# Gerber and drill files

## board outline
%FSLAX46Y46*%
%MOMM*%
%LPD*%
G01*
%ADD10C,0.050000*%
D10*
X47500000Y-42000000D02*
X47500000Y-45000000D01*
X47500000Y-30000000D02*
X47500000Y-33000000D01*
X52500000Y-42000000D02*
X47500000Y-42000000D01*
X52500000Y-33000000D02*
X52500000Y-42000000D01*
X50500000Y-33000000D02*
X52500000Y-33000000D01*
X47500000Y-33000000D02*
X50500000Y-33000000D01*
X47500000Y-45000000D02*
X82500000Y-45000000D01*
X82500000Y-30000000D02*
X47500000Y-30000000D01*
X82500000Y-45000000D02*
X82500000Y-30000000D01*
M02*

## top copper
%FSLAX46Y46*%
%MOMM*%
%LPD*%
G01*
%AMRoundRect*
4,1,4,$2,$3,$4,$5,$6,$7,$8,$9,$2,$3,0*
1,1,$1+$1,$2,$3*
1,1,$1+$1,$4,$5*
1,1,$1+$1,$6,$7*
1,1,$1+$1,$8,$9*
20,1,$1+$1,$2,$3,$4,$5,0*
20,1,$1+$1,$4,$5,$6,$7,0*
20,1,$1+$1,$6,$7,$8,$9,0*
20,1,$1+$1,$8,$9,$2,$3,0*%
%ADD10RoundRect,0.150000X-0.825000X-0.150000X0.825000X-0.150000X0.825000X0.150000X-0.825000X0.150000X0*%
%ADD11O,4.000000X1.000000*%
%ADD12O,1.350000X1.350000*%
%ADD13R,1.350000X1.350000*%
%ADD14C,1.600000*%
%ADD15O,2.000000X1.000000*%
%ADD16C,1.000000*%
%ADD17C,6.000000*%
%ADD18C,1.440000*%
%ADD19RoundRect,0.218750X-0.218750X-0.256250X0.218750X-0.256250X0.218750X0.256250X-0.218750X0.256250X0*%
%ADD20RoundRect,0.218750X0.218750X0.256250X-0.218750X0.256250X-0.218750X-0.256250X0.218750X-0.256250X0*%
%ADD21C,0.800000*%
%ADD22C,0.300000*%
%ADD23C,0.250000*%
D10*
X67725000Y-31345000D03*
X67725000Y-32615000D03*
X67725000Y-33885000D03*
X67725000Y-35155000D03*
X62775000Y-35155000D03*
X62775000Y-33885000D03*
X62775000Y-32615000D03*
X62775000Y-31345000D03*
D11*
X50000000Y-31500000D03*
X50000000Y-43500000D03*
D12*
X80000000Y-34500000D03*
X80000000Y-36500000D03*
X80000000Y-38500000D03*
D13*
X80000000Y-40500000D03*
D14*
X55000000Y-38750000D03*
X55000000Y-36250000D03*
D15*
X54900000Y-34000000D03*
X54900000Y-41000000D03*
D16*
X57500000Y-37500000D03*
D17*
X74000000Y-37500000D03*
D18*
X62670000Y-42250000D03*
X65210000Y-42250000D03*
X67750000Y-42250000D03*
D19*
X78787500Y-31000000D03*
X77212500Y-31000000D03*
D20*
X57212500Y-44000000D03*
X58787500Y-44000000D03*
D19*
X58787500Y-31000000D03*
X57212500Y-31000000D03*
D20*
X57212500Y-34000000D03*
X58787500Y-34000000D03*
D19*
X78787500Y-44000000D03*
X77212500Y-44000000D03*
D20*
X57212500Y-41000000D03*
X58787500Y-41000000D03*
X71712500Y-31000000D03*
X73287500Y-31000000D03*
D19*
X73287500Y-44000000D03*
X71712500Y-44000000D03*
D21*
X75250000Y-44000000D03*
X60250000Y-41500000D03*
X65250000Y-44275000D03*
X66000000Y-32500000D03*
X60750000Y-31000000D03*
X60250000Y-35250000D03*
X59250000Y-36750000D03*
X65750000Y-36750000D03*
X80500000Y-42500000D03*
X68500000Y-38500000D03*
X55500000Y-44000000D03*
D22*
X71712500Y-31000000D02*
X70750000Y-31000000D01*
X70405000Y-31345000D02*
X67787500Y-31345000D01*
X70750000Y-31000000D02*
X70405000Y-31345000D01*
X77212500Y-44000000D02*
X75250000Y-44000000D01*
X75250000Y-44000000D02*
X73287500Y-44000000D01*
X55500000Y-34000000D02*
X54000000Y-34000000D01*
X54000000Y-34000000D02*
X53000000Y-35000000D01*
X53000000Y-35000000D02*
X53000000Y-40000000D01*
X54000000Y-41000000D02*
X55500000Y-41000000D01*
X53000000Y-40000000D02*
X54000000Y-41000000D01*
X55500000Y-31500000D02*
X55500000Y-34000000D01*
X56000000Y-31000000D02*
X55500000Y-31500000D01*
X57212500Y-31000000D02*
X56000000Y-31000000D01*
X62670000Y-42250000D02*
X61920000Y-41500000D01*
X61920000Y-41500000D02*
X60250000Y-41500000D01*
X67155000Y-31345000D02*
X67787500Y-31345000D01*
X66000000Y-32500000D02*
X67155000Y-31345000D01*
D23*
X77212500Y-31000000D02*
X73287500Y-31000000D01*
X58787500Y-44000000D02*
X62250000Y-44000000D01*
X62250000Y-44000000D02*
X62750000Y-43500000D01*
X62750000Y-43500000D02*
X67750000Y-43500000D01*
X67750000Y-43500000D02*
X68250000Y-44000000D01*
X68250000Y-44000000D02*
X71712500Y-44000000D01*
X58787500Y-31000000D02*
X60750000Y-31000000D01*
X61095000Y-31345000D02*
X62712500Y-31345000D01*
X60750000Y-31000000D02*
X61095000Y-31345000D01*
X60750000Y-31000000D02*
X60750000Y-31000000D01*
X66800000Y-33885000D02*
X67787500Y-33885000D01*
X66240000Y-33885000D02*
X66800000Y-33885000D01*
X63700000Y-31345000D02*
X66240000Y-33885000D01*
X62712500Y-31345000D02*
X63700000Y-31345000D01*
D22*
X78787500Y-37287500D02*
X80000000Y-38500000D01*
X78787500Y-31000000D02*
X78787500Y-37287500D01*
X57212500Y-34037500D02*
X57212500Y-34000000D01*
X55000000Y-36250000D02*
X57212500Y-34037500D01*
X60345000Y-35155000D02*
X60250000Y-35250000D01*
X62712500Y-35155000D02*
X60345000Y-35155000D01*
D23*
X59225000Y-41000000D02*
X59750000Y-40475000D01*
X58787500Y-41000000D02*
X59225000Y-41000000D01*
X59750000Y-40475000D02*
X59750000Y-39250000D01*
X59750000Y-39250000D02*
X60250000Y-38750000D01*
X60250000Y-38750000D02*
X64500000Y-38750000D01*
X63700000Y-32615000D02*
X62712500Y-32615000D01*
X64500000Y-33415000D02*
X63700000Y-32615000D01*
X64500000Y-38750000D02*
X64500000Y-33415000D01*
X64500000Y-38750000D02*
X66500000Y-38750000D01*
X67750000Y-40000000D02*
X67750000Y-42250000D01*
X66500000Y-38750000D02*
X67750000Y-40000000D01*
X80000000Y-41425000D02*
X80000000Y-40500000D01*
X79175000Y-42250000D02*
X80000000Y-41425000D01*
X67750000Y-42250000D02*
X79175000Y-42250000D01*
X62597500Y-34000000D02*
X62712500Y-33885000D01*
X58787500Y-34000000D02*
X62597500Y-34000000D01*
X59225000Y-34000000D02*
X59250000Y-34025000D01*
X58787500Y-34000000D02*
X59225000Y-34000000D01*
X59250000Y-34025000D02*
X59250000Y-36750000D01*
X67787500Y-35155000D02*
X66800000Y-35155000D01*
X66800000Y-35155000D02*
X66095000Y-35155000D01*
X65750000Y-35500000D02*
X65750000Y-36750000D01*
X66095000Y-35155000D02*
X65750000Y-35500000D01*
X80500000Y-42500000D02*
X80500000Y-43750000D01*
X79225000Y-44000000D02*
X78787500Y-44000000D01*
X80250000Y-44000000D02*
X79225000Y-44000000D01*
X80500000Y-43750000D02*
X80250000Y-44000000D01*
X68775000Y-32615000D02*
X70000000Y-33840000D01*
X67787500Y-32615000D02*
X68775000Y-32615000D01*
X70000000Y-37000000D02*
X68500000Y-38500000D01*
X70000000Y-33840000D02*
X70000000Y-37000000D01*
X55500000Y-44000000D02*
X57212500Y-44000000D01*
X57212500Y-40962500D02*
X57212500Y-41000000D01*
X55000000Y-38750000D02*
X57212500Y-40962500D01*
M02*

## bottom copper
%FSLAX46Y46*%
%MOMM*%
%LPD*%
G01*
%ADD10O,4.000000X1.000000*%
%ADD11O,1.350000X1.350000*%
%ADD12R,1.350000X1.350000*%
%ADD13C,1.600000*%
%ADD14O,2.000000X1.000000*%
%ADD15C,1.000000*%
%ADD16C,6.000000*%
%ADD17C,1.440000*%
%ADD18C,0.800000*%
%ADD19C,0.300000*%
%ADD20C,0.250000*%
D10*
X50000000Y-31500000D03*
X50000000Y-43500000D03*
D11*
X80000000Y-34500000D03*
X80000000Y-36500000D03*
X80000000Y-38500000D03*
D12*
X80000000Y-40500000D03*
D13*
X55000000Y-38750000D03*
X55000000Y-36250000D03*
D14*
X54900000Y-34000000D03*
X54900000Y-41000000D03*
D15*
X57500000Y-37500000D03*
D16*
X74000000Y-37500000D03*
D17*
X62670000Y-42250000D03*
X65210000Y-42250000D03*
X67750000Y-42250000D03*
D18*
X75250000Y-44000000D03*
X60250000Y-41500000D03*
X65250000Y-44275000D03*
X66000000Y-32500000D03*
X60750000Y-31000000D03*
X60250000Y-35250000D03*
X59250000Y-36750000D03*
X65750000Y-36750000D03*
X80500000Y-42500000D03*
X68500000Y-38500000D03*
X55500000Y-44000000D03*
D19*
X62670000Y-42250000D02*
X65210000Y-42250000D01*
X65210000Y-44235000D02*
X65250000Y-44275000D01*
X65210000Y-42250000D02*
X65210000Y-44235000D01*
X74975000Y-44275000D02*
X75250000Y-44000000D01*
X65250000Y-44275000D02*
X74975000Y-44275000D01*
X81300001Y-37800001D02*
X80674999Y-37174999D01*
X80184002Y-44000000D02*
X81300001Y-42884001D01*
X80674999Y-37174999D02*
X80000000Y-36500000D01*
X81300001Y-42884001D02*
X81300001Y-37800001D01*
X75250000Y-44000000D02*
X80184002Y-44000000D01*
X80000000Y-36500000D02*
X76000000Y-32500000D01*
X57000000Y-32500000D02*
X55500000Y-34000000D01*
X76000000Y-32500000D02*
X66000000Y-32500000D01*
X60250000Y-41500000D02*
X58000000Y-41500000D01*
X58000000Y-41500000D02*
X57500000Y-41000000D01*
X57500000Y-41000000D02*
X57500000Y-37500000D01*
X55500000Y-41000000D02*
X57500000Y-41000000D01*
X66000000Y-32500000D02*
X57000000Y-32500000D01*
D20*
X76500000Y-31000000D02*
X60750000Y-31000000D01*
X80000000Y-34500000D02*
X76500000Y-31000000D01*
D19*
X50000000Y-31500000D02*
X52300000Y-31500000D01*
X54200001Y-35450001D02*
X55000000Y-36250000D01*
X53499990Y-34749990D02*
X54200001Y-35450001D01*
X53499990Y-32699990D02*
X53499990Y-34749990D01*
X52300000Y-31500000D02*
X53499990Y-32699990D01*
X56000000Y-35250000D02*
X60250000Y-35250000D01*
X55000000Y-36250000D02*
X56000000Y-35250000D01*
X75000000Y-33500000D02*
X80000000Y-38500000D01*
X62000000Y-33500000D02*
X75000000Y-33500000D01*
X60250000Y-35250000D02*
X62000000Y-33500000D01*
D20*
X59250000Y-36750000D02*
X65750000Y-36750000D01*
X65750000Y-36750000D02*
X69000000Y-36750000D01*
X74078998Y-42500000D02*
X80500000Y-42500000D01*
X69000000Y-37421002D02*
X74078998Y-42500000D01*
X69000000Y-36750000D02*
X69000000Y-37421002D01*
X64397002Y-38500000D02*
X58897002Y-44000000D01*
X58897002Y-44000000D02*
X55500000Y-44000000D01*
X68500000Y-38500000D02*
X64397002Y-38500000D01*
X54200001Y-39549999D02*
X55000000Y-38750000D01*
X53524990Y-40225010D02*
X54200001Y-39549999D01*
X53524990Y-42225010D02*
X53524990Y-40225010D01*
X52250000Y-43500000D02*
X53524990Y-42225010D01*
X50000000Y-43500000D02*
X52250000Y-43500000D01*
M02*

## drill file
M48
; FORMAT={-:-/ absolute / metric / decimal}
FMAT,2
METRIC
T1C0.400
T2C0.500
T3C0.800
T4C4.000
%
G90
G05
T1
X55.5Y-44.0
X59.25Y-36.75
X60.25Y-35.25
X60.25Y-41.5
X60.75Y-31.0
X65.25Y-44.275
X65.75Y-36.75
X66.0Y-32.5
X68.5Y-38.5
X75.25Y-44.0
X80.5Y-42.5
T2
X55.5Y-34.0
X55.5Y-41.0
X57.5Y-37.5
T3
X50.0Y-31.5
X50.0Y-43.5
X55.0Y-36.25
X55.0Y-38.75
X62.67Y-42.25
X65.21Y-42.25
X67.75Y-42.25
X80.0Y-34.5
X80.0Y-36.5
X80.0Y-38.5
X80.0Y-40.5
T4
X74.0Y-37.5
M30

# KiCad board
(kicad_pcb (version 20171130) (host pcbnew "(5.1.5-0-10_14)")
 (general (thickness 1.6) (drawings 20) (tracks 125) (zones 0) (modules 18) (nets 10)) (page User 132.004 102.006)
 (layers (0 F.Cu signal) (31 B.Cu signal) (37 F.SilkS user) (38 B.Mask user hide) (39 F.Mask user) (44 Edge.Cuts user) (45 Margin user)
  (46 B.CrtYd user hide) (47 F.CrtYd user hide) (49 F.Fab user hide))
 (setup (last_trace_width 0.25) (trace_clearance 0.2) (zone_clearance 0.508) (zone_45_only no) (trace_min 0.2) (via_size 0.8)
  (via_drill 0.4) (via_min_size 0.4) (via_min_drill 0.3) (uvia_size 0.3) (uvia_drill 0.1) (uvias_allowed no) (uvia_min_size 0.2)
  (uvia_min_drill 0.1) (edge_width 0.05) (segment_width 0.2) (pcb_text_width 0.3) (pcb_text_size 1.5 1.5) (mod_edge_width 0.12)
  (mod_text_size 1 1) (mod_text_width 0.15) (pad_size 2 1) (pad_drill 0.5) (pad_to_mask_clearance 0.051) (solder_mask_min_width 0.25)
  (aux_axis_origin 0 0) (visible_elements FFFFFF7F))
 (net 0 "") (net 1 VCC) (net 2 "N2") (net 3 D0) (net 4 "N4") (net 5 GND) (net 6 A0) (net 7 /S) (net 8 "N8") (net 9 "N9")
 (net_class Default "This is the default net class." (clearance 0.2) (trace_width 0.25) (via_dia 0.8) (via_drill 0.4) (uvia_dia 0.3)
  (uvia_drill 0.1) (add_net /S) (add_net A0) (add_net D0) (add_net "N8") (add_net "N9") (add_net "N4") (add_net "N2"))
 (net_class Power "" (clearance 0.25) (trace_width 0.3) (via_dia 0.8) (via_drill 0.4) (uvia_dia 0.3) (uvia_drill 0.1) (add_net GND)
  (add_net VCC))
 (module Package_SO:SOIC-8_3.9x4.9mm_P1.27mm (layer F.Cu) (at 65.25 33.25)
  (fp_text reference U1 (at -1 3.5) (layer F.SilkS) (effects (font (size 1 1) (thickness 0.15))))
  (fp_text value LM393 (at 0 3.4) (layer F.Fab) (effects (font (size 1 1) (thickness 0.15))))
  (pad 8 smd roundrect (at 2.475 -1.905) (size 1.95 0.6) (layers F.Cu F.Paste F.Mask) (roundrect_rratio 0.25) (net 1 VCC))
  (pad 7 smd roundrect (at 2.475 -0.635) (size 1.95 0.6) (layers F.Cu F.Paste F.Mask) (roundrect_rratio 0.25) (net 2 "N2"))
  (pad 6 smd roundrect (at 2.475 0.635) (size 1.95 0.6) (layers F.Cu F.Paste F.Mask) (roundrect_rratio 0.25) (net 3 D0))
  (pad 5 smd roundrect (at 2.475 1.905) (size 1.95 0.6) (layers F.Cu F.Paste F.Mask) (roundrect_rratio 0.25) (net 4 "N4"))
  (pad 4 smd roundrect (at -2.475 1.905) (size 1.95 0.6) (layers F.Cu F.Paste F.Mask) (roundrect_rratio 0.25) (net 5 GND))
  (pad 3 smd roundrect (at -2.475 0.635) (size 1.95 0.6) (layers F.Cu F.Paste F.Mask) (roundrect_rratio 0.25) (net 4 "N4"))
  (pad 2 smd roundrect (at -2.475 -0.635) (size 1.95 0.6) (layers F.Cu F.Paste F.Mask) (roundrect_rratio 0.25) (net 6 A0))
  (pad 1 smd roundrect (at -2.475 -1.905) (size 1.95 0.6) (layers F.Cu F.Paste F.Mask) (roundrect_rratio 0.25) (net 3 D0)))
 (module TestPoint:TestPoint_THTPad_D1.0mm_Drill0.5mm (layer F.Cu) (at 50 31.5)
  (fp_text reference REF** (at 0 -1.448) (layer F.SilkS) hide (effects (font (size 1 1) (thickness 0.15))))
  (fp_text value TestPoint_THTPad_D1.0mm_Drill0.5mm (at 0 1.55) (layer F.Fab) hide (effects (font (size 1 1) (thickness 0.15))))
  (pad G thru_hole oval (at 0 0) (size 4 1) (drill 0.8) (layers *.Cu *.Mask) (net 5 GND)))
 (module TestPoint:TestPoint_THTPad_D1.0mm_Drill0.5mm (layer F.Cu) (at 50 43.5)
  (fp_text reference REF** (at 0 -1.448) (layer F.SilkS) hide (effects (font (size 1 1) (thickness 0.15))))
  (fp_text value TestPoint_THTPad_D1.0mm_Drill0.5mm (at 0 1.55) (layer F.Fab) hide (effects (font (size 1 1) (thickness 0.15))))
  (pad S thru_hole oval (at 0 0) (size 4 1) (drill 0.8) (layers *.Cu *.Mask) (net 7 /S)))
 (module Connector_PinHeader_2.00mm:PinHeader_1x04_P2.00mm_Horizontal (layer F.Cu) (at 80 34.5)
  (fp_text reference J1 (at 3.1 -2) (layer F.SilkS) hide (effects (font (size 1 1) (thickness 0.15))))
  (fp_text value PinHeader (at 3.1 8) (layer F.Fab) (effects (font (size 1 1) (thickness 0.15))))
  (pad 4 thru_hole oval (at 0 0 180) (size 1.35 1.35) (drill 0.8) (layers *.Cu *.Mask) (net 3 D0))
  (pad 3 thru_hole oval (at 0 2 180) (size 1.35 1.35) (drill 0.8) (layers *.Cu *.Mask) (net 1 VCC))
  (pad 2 thru_hole oval (at 0 4 180) (size 1.35 1.35) (drill 0.8) (layers *.Cu *.Mask) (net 5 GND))
  (pad 1 thru_hole rect (at 0 6 180) (size 1.35 1.35) (drill 0.8) (layers *.Cu *.Mask) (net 6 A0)))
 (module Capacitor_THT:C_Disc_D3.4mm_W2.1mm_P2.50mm (layer F.Cu) (at 55 36.25 270)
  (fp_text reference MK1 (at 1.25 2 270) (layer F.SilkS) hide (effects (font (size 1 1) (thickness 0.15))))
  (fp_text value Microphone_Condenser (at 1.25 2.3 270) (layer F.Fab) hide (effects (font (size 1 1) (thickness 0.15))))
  (pad 2 thru_hole circle (at 2.5 0 270) (size 1.6 1.6) (drill 0.8) (layers *.Cu *.Mask) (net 7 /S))
  (pad 1 thru_hole circle (at 0 0 270) (size 1.6 1.6) (drill 0.8) (layers *.Cu *.Mask) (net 5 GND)))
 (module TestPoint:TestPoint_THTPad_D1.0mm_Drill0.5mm (layer F.Cu) (at 55.5 34)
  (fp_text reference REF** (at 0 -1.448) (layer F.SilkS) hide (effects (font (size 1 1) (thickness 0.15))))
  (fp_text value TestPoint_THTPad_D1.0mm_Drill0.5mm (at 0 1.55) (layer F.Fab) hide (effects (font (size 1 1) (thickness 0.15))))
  (pad + thru_hole oval (at 0 0) (size 2 1) (drill 0.5 (offset -0.6 0)) (layers *.Cu *.Mask) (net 1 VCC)))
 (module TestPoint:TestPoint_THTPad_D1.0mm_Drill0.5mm (layer F.Cu) (at 55.5 41)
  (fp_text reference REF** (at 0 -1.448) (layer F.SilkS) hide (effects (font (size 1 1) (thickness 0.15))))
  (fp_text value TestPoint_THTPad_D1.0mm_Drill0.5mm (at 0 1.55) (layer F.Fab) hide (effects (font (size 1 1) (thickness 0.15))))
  (pad + thru_hole oval (at 0 0) (size 2 1) (drill 0.5 (offset -0.6 0)) (layers *.Cu *.Mask) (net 1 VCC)))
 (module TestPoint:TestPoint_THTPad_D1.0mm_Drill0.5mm (layer F.Cu) (at 57.5 37.5)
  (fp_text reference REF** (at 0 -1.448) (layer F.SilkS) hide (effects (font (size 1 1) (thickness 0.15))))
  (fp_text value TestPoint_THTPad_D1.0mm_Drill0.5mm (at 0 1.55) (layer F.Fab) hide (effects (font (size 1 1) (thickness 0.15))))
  (pad + thru_hole circle (at 0 0) (size 1 1) (drill 0.5) (layers *.Cu *.Mask) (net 1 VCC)))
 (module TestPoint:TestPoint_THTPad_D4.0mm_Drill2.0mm (layer F.Cu) (at 74 37.5)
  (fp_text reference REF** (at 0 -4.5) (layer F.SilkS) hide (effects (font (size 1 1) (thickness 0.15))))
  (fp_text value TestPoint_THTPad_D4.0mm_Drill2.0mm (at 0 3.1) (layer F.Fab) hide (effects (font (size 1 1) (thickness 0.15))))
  (pad "" thru_hole circle (at 0 0) (size 6 6) (drill 4) (layers *.Cu *.Mask)))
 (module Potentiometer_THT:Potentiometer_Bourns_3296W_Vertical (layer F.Cu) (at 67.75 42.25)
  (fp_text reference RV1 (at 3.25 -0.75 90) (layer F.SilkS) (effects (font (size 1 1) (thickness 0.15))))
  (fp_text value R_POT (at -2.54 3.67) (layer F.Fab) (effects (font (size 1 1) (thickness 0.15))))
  (pad 3 thru_hole circle (at -5.08 0) (size 1.44 1.44) (drill 0.8) (layers *.Cu *.Mask) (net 1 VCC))
  (pad 2 thru_hole circle (at -2.54 0) (size 1.44 1.44) (drill 0.8) (layers *.Cu *.Mask) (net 1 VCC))
  (pad 1 thru_hole circle (at 0 0) (size 1.44 1.44) (drill 0.8) (layers *.Cu *.Mask) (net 6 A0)))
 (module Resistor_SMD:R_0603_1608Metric (layer F.Cu) (at 78 31)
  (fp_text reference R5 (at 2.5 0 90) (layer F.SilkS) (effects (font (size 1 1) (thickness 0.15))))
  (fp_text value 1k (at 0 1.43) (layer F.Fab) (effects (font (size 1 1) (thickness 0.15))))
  (pad 2 smd roundrect (at 0.7875 0) (size 0.875 0.95) (layers F.Cu F.Paste F.Mask) (roundrect_rratio 0.25) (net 5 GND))
  (pad 1 smd roundrect (at -0.7875 0) (size 0.875 0.95) (layers F.Cu F.Paste F.Mask) (roundrect_rratio 0.25) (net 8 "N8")))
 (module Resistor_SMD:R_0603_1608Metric (layer F.Cu) (at 58 44 180)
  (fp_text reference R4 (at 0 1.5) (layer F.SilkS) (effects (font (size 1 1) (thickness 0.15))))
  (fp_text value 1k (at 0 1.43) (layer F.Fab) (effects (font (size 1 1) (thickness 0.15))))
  (pad 2 smd roundrect (at 0.7875 0 180) (size 0.875 0.95) (layers F.Cu F.Paste F.Mask) (roundrect_rratio 0.25) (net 2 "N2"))
  (pad 1 smd roundrect (at -0.7875 0 180) (size 0.875 0.95) (layers F.Cu F.Paste F.Mask) (roundrect_rratio 0.25) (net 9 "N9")))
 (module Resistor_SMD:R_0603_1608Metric (layer F.Cu) (at 58 31)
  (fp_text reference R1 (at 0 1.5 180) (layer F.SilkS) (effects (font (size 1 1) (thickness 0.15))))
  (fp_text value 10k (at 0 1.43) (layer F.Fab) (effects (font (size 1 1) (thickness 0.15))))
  (pad 2 smd roundrect (at 0.7875 0) (size 0.875 0.95) (layers F.Cu F.Paste F.Mask) (roundrect_rratio 0.25) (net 3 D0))
  (pad 1 smd roundrect (at -0.7875 0) (size 0.875 0.95) (layers F.Cu F.Paste F.Mask) (roundrect_rratio 0.25) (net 1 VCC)))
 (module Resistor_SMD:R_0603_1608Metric (layer F.Cu) (at 58 34 180)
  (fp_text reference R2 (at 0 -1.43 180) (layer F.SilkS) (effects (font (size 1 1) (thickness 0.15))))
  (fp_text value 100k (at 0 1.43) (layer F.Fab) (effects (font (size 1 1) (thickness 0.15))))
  (pad 2 smd roundrect (at 0.7875 0 180) (size 0.875 0.95) (layers F.Cu F.Paste F.Mask) (roundrect_rratio 0.25) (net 5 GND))
  (pad 1 smd roundrect (at -0.7875 0 180) (size 0.875 0.95) (layers F.Cu F.Paste F.Mask) (roundrect_rratio 0.25) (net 4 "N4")))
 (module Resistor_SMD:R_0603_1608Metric (layer F.Cu) (at 78 44)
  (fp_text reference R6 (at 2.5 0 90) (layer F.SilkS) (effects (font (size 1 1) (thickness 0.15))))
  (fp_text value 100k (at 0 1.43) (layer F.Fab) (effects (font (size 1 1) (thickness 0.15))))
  (pad 2 smd roundrect (at 0.7875 0) (size 0.875 0.95) (layers F.Cu F.Paste F.Mask) (roundrect_rratio 0.25) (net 4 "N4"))
  (pad 1 smd roundrect (at -0.7875 0) (size 0.875 0.95) (layers F.Cu F.Paste F.Mask) (roundrect_rratio 0.25) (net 1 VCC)))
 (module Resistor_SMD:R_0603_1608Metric (layer F.Cu) (at 58 41 180)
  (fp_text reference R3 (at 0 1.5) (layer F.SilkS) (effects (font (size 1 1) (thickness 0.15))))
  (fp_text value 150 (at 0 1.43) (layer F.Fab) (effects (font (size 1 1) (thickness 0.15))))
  (pad 2 smd roundrect (at 0.7875 0 180) (size 0.875 0.95) (layers F.Cu F.Paste F.Mask) (roundrect_rratio 0.25) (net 7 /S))
  (pad 1 smd roundrect (at -0.7875 0 180) (size 0.875 0.95) (layers F.Cu F.Paste F.Mask) (roundrect_rratio 0.25) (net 6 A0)))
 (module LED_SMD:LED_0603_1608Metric (layer F.Cu) (at 72.5 31 180)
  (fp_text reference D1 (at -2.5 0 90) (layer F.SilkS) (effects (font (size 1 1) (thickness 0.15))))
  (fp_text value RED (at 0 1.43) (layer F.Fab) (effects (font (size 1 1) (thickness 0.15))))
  (pad 2 smd roundrect (at 0.7875 0 180) (size 0.875 0.95) (layers F.Cu F.Paste F.Mask) (roundrect_rratio 0.25) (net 1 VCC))
  (pad 1 smd roundrect (at -0.7875 0 180) (size 0.875 0.95) (layers F.Cu F.Paste F.Mask) (roundrect_rratio 0.25) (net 8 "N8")))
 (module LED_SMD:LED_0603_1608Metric (layer F.Cu) (at 72.5 44)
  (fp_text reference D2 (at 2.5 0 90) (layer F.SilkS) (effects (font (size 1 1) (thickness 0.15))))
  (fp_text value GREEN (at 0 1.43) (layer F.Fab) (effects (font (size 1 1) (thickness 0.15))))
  (pad 2 smd roundrect (at 0.7875 0) (size 0.875 0.95) (layers F.Cu F.Paste F.Mask) (roundrect_rratio 0.25) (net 1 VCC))
  (pad 1 smd roundrect (at -0.7875 0) (size 0.875 0.95) (layers F.Cu F.Paste F.Mask) (roundrect_rratio 0.25) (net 9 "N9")))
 (gr_line (start 47.5 42) (end 47.5 45) (layer Edge.Cuts) (width 0.05))
 (gr_line (start 47.5 30) (end 47.5 33) (layer Edge.Cuts) (width 0.05))
 (gr_line (start 52.5 42) (end 47.5 42) (layer Edge.Cuts) (width 0.05))
 (gr_line (start 52.5 33) (end 52.5 42) (layer Edge.Cuts) (width 0.05))
 (gr_line (start 50.5 33) (end 52.5 33) (layer Edge.Cuts) (width 0.05))
 (gr_line (start 47.5 33) (end 50.5 33) (layer Edge.Cuts) (width 0.05))
 (gr_line (start 47.5 45) (end 82.5 45) (layer Edge.Cuts) (width 0.05))
 (gr_line (start 82.5 30) (end 47.5 30) (layer Edge.Cuts) (width 0.05))
 (gr_line (start 82.5 45) (end 82.5 30) (layer Edge.Cuts) (width 0.05))
 (segment (start 71.7125 31) (end 70.75 31) (width 0.3) (layer F.Cu) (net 1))
 (segment (start 70.405 31.345) (end 67.7875 31.345) (width 0.3) (layer F.Cu) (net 1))
 (segment (start 70.75 31) (end 70.405 31.345) (width 0.3) (layer F.Cu) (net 1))
 (segment (start 77.2125 44) (end 75.25 44) (width 0.3) (layer F.Cu) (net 1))
 (segment (start 75.25 44) (end 73.2875 44) (width 0.3) (layer F.Cu) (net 1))
 (via (at 75.25 44) (size 0.8) (drill 0.4) (layers F.Cu B.Cu) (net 1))
 (segment (start 55.5 34) (end 54 34) (width 0.3) (layer F.Cu) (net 1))
 (segment (start 54 34) (end 53 35) (width 0.3) (layer F.Cu) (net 1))
 (segment (start 53 35) (end 53 40) (width 0.3) (layer F.Cu) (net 1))
 (segment (start 54 41) (end 55.5 41) (width 0.3) (layer F.Cu) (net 1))
 (segment (start 53 40) (end 54 41) (width 0.3) (layer F.Cu) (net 1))
 (segment (start 55.5 31.5) (end 55.5 34) (width 0.3) (layer F.Cu) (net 1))
 (segment (start 56 31) (end 55.5 31.5) (width 0.3) (layer F.Cu) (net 1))
 (segment (start 57.2125 31) (end 56 31) (width 0.3) (layer F.Cu) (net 1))
 (segment (start 62.67 42.25) (end 61.92 41.5) (width 0.3) (layer F.Cu) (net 1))
 (via (at 60.25 41.5) (size 0.8) (drill 0.4) (layers F.Cu B.Cu) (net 1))
 (segment (start 61.92 41.5) (end 60.25 41.5) (width 0.3) (layer F.Cu) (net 1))
 (segment (start 62.67 42.25) (end 65.21 42.25) (width 0.3) (layer B.Cu) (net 1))
 (via (at 65.25 44.275) (size 0.8) (drill 0.4) (layers F.Cu B.Cu) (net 1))
 (segment (start 65.21 44.235) (end 65.25 44.275) (width 0.3) (layer B.Cu) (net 1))
 (segment (start 65.21 42.25) (end 65.21 44.235) (width 0.3) (layer B.Cu) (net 1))
 (segment (start 74.975 44.275) (end 75.25 44) (width 0.3) (layer B.Cu) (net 1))
 (segment (start 65.25 44.275) (end 74.975 44.275) (width 0.3) (layer B.Cu) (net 1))
 (segment (start 81.300001 37.800001) (end 80.674999 37.174999) (width 0.3) (layer B.Cu) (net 1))
 (segment (start 80.184002 44) (end 81.300001 42.884001) (width 0.3) (layer B.Cu) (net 1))
 (segment (start 80.674999 37.174999) (end 80 36.5) (width 0.3) (layer B.Cu) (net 1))
 (segment (start 81.300001 42.884001) (end 81.300001 37.800001) (width 0.3) (layer B.Cu) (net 1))
 (segment (start 75.25 44) (end 80.184002 44) (width 0.3) (layer B.Cu) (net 1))
 (segment (start 80 36.5) (end 76 32.5) (width 0.3) (layer B.Cu) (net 1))
 (segment (start 57 32.5) (end 55.5 34) (width 0.3) (layer B.Cu) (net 1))
 (segment (start 76 32.5) (end 66 32.5) (width 0.3) (layer B.Cu) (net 1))
 (segment (start 60.25 41.5) (end 58 41.5) (width 0.3) (layer B.Cu) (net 1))
 (segment (start 58 41.5) (end 57.5 41) (width 0.3) (layer B.Cu) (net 1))
 (segment (start 57.5 41) (end 57.5 37.5) (width 0.3) (layer B.Cu) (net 1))
 (segment (start 55.5 41) (end 57.5 41) (width 0.3) (layer B.Cu) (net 1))
 (segment (start 66 32.5) (end 57 32.5) (width 0.3) (layer B.Cu) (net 1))
 (via (at 66 32.5) (size 0.8) (drill 0.4) (layers F.Cu B.Cu) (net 1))
 (segment (start 67.155 31.345) (end 67.7875 31.345) (width 0.3) (layer F.Cu) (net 1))
 (segment (start 66 32.5) (end 67.155 31.345) (width 0.3) (layer F.Cu) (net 1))
 (segment (start 77.2125 31) (end 73.2875 31) (width 0.25) (layer F.Cu) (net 8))
 (segment (start 58.7875 44) (end 62.25 44) (width 0.25) (layer F.Cu) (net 9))
 (segment (start 62.25 44) (end 62.75 43.5) (width 0.25) (layer F.Cu) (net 9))
 (segment (start 62.75 43.5) (end 67.75 43.5) (width 0.25) (layer F.Cu) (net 9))
 (segment (start 67.75 43.5) (end 68.25 44) (width 0.25) (layer F.Cu) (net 9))
 (segment (start 68.25 44) (end 71.7125 44) (width 0.25) (layer F.Cu) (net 9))
 (segment (start 58.7875 31) (end 60.75 31) (width 0.25) (layer F.Cu) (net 3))
 (segment (start 61.095 31.345) (end 62.7125 31.345) (width 0.25) (layer F.Cu) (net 3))
 (segment (start 60.75 31) (end 61.095 31.345) (width 0.25) (layer F.Cu) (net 3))
 (segment (start 60.75 31) (end 60.75 31) (width 0.25) (layer F.Cu) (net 3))
 (via (at 60.75 31) (size 0.8) (drill 0.4) (layers F.Cu B.Cu) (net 3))
 (segment (start 66.8 33.885) (end 67.7875 33.885) (width 0.25) (layer F.Cu) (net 3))
 (segment (start 66.24 33.885) (end 66.8 33.885) (width 0.25) (layer F.Cu) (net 3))
 (segment (start 63.7 31.345) (end 66.24 33.885) (width 0.25) (layer F.Cu) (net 3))
 (segment (start 62.7125 31.345) (end 63.7 31.345) (width 0.25) (layer F.Cu) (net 3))
 (segment (start 76.5 31) (end 60.75 31) (width 0.25) (layer B.Cu) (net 3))
 (segment (start 80 34.5) (end 76.5 31) (width 0.25) (layer B.Cu) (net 3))
 (segment (start 78.7875 37.2875) (end 80 38.5) (width 0.3) (layer F.Cu) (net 5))
 (segment (start 78.7875 31) (end 78.7875 37.2875) (width 0.3) (layer F.Cu) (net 5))
 (segment (start 57.2125 34.0375) (end 57.2125 34) (width 0.3) (layer F.Cu) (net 5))
 (segment (start 55 36.25) (end 57.2125 34.0375) (width 0.3) (layer F.Cu) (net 5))
 (via (at 60.25 35.25) (size 0.8) (drill 0.4) (layers F.Cu B.Cu) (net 5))
 (segment (start 60.345 35.155) (end 60.25 35.25) (width 0.3) (layer F.Cu) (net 5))
 (segment (start 62.7125 35.155) (end 60.345 35.155) (width 0.3) (layer F.Cu) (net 5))
 (segment (start 50 31.5) (end 52.3 31.5) (width 0.3) (layer B.Cu) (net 5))
 (segment (start 54.200001 35.450001) (end 55 36.25) (width 0.3) (layer B.Cu) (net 5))
 (segment (start 53.49999 34.74999) (end 54.200001 35.450001) (width 0.3) (layer B.Cu) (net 5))
 (segment (start 53.49999 32.69999) (end 53.49999 34.74999) (width 0.3) (layer B.Cu) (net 5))
 (segment (start 52.3 31.5) (end 53.49999 32.69999) (width 0.3) (layer B.Cu) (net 5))
 (segment (start 56 35.25) (end 60.25 35.25) (width 0.3) (layer B.Cu) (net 5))
 (segment (start 55 36.25) (end 56 35.25) (width 0.3) (layer B.Cu) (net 5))
 (segment (start 75 33.5) (end 80 38.5) (width 0.3) (layer B.Cu) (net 5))
 (segment (start 62 33.5) (end 75 33.5) (width 0.3) (layer B.Cu) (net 5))
 (segment (start 60.25 35.25) (end 62 33.5) (width 0.3) (layer B.Cu) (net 5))
 (segment (start 59.225 41) (end 59.75 40.475) (width 0.25) (layer F.Cu) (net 6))
 (segment (start 58.7875 41) (end 59.225 41) (width 0.25) (layer F.Cu) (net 6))
 (segment (start 59.75 40.475) (end 59.75 39.25) (width 0.25) (layer F.Cu) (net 6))
 (segment (start 59.75 39.25) (end 60.25 38.75) (width 0.25) (layer F.Cu) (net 6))
 (segment (start 60.25 38.75) (end 64.5 38.75) (width 0.25) (layer F.Cu) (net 6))
 (segment (start 63.7 32.615) (end 62.7125 32.615) (width 0.25) (layer F.Cu) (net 6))
 (segment (start 64.5 33.415) (end 63.7 32.615) (width 0.25) (layer F.Cu) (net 6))
 (segment (start 64.5 38.75) (end 64.5 33.415) (width 0.25) (layer F.Cu) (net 6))
 (segment (start 64.5 38.75) (end 66.5 38.75) (width 0.25) (layer F.Cu) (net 6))
 (segment (start 67.75 40) (end 67.75 42.25) (width 0.25) (layer F.Cu) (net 6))
 (segment (start 66.5 38.75) (end 67.75 40) (width 0.25) (layer F.Cu) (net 6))
 (segment (start 80 41.425) (end 80 40.5) (width 0.25) (layer F.Cu) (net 6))
 (segment (start 79.175 42.25) (end 80 41.425) (width 0.25) (layer F.Cu) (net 6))
 (segment (start 67.75 42.25) (end 79.175 42.25) (width 0.25) (layer F.Cu) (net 6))
 (segment (start 62.5975 34) (end 62.7125 33.885) (width 0.25) (layer F.Cu) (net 4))
 (segment (start 58.7875 34) (end 62.5975 34) (width 0.25) (layer F.Cu) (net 4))
 (segment (start 59.225 34) (end 59.25 34.025) (width 0.25) (layer F.Cu) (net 4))
 (segment (start 58.7875 34) (end 59.225 34) (width 0.25) (layer F.Cu) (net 4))
 (via (at 59.25 36.75) (size 0.8) (drill 0.4) (layers F.Cu B.Cu) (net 4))
 (segment (start 59.25 34.025) (end 59.25 36.75) (width 0.25) (layer F.Cu) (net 4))
 (segment (start 67.7875 35.155) (end 66.8 35.155) (width 0.25) (layer F.Cu) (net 4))
 (segment (start 66.8 35.155) (end 66.095 35.155) (width 0.25) (layer F.Cu) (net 4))
 (via (at 65.75 36.75) (size 0.8) (drill 0.4) (layers F.Cu B.Cu) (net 4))
 (segment (start 65.75 35.5) (end 65.75 36.75) (width 0.25) (layer F.Cu) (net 4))
 (segment (start 66.095 35.155) (end 65.75 35.5) (width 0.25) (layer F.Cu) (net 4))
 (segment (start 59.25 36.75) (end 65.75 36.75) (width 0.25) (layer B.Cu) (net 4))
 (segment (start 65.75 36.75) (end 69 36.75) (width 0.25) (layer B.Cu) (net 4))
 (via (at 80.5 42.5) (size 0.8) (drill 0.4) (layers F.Cu B.Cu) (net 4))
 (segment (start 74.078998 42.5) (end 80.5 42.5) (width 0.25) (layer B.Cu) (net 4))
 (segment (start 69 37.421002) (end 74.078998 42.5) (width 0.25) (layer B.Cu) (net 4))
 (segment (start 69 36.75) (end 69 37.421002) (width 0.25) (layer B.Cu) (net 4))
 (segment (start 80.5 42.5) (end 80.5 43.75) (width 0.25) (layer F.Cu) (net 4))
 (segment (start 79.225 44) (end 78.7875 44) (width 0.25) (layer F.Cu) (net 4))
 (segment (start 80.25 44) (end 79.225 44) (width 0.25) (layer F.Cu) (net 4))
 (segment (start 80.5 43.75) (end 80.25 44) (width 0.25) (layer F.Cu) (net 4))
 (segment (start 68.775 32.615) (end 70 33.84) (width 0.25) (layer F.Cu) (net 2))
 (segment (start 67.7875 32.615) (end 68.775 32.615) (width 0.25) (layer F.Cu) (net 2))
 (via (at 68.5 38.5) (size 0.8) (drill 0.4) (layers F.Cu B.Cu) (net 2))
 (segment (start 70 37) (end 68.5 38.5) (width 0.25) (layer F.Cu) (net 2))
 (segment (start 70 33.84) (end 70 37) (width 0.25) (layer F.Cu) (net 2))
 (via (at 55.5 44) (size 0.8) (drill 0.4) (layers F.Cu B.Cu) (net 2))
 (segment (start 64.397002 38.5) (end 58.897002 44) (width 0.25) (layer B.Cu) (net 2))
 (segment (start 58.897002 44) (end 55.5 44) (width 0.25) (layer B.Cu) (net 2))
 (segment (start 68.5 38.5) (end 64.397002 38.5) (width 0.25) (layer B.Cu) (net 2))
 (segment (start 55.5 44) (end 57.2125 44) (width 0.25) (layer F.Cu) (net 2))
 (segment (start 57.2125 40.9625) (end 57.2125 41) (width 0.25) (layer F.Cu) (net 7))
 (segment (start 55 38.75) (end 57.2125 40.9625) (width 0.25) (layer F.Cu) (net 7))
 (segment (start 54.200001 39.549999) (end 55 38.75) (width 0.25) (layer B.Cu) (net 7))
 (segment (start 53.52499 40.22501) (end 54.200001 39.549999) (width 0.25) (layer B.Cu) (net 7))
 (segment (start 53.52499 42.22501) (end 53.52499 40.22501) (width 0.25) (layer B.Cu) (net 7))
 (segment (start 52.25 43.5) (end 53.52499 42.22501) (width 0.25) (layer B.Cu) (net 7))
 (segment (start 50 43.5) (end 52.25 43.5) (width 0.25) (layer B.Cu) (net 7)))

